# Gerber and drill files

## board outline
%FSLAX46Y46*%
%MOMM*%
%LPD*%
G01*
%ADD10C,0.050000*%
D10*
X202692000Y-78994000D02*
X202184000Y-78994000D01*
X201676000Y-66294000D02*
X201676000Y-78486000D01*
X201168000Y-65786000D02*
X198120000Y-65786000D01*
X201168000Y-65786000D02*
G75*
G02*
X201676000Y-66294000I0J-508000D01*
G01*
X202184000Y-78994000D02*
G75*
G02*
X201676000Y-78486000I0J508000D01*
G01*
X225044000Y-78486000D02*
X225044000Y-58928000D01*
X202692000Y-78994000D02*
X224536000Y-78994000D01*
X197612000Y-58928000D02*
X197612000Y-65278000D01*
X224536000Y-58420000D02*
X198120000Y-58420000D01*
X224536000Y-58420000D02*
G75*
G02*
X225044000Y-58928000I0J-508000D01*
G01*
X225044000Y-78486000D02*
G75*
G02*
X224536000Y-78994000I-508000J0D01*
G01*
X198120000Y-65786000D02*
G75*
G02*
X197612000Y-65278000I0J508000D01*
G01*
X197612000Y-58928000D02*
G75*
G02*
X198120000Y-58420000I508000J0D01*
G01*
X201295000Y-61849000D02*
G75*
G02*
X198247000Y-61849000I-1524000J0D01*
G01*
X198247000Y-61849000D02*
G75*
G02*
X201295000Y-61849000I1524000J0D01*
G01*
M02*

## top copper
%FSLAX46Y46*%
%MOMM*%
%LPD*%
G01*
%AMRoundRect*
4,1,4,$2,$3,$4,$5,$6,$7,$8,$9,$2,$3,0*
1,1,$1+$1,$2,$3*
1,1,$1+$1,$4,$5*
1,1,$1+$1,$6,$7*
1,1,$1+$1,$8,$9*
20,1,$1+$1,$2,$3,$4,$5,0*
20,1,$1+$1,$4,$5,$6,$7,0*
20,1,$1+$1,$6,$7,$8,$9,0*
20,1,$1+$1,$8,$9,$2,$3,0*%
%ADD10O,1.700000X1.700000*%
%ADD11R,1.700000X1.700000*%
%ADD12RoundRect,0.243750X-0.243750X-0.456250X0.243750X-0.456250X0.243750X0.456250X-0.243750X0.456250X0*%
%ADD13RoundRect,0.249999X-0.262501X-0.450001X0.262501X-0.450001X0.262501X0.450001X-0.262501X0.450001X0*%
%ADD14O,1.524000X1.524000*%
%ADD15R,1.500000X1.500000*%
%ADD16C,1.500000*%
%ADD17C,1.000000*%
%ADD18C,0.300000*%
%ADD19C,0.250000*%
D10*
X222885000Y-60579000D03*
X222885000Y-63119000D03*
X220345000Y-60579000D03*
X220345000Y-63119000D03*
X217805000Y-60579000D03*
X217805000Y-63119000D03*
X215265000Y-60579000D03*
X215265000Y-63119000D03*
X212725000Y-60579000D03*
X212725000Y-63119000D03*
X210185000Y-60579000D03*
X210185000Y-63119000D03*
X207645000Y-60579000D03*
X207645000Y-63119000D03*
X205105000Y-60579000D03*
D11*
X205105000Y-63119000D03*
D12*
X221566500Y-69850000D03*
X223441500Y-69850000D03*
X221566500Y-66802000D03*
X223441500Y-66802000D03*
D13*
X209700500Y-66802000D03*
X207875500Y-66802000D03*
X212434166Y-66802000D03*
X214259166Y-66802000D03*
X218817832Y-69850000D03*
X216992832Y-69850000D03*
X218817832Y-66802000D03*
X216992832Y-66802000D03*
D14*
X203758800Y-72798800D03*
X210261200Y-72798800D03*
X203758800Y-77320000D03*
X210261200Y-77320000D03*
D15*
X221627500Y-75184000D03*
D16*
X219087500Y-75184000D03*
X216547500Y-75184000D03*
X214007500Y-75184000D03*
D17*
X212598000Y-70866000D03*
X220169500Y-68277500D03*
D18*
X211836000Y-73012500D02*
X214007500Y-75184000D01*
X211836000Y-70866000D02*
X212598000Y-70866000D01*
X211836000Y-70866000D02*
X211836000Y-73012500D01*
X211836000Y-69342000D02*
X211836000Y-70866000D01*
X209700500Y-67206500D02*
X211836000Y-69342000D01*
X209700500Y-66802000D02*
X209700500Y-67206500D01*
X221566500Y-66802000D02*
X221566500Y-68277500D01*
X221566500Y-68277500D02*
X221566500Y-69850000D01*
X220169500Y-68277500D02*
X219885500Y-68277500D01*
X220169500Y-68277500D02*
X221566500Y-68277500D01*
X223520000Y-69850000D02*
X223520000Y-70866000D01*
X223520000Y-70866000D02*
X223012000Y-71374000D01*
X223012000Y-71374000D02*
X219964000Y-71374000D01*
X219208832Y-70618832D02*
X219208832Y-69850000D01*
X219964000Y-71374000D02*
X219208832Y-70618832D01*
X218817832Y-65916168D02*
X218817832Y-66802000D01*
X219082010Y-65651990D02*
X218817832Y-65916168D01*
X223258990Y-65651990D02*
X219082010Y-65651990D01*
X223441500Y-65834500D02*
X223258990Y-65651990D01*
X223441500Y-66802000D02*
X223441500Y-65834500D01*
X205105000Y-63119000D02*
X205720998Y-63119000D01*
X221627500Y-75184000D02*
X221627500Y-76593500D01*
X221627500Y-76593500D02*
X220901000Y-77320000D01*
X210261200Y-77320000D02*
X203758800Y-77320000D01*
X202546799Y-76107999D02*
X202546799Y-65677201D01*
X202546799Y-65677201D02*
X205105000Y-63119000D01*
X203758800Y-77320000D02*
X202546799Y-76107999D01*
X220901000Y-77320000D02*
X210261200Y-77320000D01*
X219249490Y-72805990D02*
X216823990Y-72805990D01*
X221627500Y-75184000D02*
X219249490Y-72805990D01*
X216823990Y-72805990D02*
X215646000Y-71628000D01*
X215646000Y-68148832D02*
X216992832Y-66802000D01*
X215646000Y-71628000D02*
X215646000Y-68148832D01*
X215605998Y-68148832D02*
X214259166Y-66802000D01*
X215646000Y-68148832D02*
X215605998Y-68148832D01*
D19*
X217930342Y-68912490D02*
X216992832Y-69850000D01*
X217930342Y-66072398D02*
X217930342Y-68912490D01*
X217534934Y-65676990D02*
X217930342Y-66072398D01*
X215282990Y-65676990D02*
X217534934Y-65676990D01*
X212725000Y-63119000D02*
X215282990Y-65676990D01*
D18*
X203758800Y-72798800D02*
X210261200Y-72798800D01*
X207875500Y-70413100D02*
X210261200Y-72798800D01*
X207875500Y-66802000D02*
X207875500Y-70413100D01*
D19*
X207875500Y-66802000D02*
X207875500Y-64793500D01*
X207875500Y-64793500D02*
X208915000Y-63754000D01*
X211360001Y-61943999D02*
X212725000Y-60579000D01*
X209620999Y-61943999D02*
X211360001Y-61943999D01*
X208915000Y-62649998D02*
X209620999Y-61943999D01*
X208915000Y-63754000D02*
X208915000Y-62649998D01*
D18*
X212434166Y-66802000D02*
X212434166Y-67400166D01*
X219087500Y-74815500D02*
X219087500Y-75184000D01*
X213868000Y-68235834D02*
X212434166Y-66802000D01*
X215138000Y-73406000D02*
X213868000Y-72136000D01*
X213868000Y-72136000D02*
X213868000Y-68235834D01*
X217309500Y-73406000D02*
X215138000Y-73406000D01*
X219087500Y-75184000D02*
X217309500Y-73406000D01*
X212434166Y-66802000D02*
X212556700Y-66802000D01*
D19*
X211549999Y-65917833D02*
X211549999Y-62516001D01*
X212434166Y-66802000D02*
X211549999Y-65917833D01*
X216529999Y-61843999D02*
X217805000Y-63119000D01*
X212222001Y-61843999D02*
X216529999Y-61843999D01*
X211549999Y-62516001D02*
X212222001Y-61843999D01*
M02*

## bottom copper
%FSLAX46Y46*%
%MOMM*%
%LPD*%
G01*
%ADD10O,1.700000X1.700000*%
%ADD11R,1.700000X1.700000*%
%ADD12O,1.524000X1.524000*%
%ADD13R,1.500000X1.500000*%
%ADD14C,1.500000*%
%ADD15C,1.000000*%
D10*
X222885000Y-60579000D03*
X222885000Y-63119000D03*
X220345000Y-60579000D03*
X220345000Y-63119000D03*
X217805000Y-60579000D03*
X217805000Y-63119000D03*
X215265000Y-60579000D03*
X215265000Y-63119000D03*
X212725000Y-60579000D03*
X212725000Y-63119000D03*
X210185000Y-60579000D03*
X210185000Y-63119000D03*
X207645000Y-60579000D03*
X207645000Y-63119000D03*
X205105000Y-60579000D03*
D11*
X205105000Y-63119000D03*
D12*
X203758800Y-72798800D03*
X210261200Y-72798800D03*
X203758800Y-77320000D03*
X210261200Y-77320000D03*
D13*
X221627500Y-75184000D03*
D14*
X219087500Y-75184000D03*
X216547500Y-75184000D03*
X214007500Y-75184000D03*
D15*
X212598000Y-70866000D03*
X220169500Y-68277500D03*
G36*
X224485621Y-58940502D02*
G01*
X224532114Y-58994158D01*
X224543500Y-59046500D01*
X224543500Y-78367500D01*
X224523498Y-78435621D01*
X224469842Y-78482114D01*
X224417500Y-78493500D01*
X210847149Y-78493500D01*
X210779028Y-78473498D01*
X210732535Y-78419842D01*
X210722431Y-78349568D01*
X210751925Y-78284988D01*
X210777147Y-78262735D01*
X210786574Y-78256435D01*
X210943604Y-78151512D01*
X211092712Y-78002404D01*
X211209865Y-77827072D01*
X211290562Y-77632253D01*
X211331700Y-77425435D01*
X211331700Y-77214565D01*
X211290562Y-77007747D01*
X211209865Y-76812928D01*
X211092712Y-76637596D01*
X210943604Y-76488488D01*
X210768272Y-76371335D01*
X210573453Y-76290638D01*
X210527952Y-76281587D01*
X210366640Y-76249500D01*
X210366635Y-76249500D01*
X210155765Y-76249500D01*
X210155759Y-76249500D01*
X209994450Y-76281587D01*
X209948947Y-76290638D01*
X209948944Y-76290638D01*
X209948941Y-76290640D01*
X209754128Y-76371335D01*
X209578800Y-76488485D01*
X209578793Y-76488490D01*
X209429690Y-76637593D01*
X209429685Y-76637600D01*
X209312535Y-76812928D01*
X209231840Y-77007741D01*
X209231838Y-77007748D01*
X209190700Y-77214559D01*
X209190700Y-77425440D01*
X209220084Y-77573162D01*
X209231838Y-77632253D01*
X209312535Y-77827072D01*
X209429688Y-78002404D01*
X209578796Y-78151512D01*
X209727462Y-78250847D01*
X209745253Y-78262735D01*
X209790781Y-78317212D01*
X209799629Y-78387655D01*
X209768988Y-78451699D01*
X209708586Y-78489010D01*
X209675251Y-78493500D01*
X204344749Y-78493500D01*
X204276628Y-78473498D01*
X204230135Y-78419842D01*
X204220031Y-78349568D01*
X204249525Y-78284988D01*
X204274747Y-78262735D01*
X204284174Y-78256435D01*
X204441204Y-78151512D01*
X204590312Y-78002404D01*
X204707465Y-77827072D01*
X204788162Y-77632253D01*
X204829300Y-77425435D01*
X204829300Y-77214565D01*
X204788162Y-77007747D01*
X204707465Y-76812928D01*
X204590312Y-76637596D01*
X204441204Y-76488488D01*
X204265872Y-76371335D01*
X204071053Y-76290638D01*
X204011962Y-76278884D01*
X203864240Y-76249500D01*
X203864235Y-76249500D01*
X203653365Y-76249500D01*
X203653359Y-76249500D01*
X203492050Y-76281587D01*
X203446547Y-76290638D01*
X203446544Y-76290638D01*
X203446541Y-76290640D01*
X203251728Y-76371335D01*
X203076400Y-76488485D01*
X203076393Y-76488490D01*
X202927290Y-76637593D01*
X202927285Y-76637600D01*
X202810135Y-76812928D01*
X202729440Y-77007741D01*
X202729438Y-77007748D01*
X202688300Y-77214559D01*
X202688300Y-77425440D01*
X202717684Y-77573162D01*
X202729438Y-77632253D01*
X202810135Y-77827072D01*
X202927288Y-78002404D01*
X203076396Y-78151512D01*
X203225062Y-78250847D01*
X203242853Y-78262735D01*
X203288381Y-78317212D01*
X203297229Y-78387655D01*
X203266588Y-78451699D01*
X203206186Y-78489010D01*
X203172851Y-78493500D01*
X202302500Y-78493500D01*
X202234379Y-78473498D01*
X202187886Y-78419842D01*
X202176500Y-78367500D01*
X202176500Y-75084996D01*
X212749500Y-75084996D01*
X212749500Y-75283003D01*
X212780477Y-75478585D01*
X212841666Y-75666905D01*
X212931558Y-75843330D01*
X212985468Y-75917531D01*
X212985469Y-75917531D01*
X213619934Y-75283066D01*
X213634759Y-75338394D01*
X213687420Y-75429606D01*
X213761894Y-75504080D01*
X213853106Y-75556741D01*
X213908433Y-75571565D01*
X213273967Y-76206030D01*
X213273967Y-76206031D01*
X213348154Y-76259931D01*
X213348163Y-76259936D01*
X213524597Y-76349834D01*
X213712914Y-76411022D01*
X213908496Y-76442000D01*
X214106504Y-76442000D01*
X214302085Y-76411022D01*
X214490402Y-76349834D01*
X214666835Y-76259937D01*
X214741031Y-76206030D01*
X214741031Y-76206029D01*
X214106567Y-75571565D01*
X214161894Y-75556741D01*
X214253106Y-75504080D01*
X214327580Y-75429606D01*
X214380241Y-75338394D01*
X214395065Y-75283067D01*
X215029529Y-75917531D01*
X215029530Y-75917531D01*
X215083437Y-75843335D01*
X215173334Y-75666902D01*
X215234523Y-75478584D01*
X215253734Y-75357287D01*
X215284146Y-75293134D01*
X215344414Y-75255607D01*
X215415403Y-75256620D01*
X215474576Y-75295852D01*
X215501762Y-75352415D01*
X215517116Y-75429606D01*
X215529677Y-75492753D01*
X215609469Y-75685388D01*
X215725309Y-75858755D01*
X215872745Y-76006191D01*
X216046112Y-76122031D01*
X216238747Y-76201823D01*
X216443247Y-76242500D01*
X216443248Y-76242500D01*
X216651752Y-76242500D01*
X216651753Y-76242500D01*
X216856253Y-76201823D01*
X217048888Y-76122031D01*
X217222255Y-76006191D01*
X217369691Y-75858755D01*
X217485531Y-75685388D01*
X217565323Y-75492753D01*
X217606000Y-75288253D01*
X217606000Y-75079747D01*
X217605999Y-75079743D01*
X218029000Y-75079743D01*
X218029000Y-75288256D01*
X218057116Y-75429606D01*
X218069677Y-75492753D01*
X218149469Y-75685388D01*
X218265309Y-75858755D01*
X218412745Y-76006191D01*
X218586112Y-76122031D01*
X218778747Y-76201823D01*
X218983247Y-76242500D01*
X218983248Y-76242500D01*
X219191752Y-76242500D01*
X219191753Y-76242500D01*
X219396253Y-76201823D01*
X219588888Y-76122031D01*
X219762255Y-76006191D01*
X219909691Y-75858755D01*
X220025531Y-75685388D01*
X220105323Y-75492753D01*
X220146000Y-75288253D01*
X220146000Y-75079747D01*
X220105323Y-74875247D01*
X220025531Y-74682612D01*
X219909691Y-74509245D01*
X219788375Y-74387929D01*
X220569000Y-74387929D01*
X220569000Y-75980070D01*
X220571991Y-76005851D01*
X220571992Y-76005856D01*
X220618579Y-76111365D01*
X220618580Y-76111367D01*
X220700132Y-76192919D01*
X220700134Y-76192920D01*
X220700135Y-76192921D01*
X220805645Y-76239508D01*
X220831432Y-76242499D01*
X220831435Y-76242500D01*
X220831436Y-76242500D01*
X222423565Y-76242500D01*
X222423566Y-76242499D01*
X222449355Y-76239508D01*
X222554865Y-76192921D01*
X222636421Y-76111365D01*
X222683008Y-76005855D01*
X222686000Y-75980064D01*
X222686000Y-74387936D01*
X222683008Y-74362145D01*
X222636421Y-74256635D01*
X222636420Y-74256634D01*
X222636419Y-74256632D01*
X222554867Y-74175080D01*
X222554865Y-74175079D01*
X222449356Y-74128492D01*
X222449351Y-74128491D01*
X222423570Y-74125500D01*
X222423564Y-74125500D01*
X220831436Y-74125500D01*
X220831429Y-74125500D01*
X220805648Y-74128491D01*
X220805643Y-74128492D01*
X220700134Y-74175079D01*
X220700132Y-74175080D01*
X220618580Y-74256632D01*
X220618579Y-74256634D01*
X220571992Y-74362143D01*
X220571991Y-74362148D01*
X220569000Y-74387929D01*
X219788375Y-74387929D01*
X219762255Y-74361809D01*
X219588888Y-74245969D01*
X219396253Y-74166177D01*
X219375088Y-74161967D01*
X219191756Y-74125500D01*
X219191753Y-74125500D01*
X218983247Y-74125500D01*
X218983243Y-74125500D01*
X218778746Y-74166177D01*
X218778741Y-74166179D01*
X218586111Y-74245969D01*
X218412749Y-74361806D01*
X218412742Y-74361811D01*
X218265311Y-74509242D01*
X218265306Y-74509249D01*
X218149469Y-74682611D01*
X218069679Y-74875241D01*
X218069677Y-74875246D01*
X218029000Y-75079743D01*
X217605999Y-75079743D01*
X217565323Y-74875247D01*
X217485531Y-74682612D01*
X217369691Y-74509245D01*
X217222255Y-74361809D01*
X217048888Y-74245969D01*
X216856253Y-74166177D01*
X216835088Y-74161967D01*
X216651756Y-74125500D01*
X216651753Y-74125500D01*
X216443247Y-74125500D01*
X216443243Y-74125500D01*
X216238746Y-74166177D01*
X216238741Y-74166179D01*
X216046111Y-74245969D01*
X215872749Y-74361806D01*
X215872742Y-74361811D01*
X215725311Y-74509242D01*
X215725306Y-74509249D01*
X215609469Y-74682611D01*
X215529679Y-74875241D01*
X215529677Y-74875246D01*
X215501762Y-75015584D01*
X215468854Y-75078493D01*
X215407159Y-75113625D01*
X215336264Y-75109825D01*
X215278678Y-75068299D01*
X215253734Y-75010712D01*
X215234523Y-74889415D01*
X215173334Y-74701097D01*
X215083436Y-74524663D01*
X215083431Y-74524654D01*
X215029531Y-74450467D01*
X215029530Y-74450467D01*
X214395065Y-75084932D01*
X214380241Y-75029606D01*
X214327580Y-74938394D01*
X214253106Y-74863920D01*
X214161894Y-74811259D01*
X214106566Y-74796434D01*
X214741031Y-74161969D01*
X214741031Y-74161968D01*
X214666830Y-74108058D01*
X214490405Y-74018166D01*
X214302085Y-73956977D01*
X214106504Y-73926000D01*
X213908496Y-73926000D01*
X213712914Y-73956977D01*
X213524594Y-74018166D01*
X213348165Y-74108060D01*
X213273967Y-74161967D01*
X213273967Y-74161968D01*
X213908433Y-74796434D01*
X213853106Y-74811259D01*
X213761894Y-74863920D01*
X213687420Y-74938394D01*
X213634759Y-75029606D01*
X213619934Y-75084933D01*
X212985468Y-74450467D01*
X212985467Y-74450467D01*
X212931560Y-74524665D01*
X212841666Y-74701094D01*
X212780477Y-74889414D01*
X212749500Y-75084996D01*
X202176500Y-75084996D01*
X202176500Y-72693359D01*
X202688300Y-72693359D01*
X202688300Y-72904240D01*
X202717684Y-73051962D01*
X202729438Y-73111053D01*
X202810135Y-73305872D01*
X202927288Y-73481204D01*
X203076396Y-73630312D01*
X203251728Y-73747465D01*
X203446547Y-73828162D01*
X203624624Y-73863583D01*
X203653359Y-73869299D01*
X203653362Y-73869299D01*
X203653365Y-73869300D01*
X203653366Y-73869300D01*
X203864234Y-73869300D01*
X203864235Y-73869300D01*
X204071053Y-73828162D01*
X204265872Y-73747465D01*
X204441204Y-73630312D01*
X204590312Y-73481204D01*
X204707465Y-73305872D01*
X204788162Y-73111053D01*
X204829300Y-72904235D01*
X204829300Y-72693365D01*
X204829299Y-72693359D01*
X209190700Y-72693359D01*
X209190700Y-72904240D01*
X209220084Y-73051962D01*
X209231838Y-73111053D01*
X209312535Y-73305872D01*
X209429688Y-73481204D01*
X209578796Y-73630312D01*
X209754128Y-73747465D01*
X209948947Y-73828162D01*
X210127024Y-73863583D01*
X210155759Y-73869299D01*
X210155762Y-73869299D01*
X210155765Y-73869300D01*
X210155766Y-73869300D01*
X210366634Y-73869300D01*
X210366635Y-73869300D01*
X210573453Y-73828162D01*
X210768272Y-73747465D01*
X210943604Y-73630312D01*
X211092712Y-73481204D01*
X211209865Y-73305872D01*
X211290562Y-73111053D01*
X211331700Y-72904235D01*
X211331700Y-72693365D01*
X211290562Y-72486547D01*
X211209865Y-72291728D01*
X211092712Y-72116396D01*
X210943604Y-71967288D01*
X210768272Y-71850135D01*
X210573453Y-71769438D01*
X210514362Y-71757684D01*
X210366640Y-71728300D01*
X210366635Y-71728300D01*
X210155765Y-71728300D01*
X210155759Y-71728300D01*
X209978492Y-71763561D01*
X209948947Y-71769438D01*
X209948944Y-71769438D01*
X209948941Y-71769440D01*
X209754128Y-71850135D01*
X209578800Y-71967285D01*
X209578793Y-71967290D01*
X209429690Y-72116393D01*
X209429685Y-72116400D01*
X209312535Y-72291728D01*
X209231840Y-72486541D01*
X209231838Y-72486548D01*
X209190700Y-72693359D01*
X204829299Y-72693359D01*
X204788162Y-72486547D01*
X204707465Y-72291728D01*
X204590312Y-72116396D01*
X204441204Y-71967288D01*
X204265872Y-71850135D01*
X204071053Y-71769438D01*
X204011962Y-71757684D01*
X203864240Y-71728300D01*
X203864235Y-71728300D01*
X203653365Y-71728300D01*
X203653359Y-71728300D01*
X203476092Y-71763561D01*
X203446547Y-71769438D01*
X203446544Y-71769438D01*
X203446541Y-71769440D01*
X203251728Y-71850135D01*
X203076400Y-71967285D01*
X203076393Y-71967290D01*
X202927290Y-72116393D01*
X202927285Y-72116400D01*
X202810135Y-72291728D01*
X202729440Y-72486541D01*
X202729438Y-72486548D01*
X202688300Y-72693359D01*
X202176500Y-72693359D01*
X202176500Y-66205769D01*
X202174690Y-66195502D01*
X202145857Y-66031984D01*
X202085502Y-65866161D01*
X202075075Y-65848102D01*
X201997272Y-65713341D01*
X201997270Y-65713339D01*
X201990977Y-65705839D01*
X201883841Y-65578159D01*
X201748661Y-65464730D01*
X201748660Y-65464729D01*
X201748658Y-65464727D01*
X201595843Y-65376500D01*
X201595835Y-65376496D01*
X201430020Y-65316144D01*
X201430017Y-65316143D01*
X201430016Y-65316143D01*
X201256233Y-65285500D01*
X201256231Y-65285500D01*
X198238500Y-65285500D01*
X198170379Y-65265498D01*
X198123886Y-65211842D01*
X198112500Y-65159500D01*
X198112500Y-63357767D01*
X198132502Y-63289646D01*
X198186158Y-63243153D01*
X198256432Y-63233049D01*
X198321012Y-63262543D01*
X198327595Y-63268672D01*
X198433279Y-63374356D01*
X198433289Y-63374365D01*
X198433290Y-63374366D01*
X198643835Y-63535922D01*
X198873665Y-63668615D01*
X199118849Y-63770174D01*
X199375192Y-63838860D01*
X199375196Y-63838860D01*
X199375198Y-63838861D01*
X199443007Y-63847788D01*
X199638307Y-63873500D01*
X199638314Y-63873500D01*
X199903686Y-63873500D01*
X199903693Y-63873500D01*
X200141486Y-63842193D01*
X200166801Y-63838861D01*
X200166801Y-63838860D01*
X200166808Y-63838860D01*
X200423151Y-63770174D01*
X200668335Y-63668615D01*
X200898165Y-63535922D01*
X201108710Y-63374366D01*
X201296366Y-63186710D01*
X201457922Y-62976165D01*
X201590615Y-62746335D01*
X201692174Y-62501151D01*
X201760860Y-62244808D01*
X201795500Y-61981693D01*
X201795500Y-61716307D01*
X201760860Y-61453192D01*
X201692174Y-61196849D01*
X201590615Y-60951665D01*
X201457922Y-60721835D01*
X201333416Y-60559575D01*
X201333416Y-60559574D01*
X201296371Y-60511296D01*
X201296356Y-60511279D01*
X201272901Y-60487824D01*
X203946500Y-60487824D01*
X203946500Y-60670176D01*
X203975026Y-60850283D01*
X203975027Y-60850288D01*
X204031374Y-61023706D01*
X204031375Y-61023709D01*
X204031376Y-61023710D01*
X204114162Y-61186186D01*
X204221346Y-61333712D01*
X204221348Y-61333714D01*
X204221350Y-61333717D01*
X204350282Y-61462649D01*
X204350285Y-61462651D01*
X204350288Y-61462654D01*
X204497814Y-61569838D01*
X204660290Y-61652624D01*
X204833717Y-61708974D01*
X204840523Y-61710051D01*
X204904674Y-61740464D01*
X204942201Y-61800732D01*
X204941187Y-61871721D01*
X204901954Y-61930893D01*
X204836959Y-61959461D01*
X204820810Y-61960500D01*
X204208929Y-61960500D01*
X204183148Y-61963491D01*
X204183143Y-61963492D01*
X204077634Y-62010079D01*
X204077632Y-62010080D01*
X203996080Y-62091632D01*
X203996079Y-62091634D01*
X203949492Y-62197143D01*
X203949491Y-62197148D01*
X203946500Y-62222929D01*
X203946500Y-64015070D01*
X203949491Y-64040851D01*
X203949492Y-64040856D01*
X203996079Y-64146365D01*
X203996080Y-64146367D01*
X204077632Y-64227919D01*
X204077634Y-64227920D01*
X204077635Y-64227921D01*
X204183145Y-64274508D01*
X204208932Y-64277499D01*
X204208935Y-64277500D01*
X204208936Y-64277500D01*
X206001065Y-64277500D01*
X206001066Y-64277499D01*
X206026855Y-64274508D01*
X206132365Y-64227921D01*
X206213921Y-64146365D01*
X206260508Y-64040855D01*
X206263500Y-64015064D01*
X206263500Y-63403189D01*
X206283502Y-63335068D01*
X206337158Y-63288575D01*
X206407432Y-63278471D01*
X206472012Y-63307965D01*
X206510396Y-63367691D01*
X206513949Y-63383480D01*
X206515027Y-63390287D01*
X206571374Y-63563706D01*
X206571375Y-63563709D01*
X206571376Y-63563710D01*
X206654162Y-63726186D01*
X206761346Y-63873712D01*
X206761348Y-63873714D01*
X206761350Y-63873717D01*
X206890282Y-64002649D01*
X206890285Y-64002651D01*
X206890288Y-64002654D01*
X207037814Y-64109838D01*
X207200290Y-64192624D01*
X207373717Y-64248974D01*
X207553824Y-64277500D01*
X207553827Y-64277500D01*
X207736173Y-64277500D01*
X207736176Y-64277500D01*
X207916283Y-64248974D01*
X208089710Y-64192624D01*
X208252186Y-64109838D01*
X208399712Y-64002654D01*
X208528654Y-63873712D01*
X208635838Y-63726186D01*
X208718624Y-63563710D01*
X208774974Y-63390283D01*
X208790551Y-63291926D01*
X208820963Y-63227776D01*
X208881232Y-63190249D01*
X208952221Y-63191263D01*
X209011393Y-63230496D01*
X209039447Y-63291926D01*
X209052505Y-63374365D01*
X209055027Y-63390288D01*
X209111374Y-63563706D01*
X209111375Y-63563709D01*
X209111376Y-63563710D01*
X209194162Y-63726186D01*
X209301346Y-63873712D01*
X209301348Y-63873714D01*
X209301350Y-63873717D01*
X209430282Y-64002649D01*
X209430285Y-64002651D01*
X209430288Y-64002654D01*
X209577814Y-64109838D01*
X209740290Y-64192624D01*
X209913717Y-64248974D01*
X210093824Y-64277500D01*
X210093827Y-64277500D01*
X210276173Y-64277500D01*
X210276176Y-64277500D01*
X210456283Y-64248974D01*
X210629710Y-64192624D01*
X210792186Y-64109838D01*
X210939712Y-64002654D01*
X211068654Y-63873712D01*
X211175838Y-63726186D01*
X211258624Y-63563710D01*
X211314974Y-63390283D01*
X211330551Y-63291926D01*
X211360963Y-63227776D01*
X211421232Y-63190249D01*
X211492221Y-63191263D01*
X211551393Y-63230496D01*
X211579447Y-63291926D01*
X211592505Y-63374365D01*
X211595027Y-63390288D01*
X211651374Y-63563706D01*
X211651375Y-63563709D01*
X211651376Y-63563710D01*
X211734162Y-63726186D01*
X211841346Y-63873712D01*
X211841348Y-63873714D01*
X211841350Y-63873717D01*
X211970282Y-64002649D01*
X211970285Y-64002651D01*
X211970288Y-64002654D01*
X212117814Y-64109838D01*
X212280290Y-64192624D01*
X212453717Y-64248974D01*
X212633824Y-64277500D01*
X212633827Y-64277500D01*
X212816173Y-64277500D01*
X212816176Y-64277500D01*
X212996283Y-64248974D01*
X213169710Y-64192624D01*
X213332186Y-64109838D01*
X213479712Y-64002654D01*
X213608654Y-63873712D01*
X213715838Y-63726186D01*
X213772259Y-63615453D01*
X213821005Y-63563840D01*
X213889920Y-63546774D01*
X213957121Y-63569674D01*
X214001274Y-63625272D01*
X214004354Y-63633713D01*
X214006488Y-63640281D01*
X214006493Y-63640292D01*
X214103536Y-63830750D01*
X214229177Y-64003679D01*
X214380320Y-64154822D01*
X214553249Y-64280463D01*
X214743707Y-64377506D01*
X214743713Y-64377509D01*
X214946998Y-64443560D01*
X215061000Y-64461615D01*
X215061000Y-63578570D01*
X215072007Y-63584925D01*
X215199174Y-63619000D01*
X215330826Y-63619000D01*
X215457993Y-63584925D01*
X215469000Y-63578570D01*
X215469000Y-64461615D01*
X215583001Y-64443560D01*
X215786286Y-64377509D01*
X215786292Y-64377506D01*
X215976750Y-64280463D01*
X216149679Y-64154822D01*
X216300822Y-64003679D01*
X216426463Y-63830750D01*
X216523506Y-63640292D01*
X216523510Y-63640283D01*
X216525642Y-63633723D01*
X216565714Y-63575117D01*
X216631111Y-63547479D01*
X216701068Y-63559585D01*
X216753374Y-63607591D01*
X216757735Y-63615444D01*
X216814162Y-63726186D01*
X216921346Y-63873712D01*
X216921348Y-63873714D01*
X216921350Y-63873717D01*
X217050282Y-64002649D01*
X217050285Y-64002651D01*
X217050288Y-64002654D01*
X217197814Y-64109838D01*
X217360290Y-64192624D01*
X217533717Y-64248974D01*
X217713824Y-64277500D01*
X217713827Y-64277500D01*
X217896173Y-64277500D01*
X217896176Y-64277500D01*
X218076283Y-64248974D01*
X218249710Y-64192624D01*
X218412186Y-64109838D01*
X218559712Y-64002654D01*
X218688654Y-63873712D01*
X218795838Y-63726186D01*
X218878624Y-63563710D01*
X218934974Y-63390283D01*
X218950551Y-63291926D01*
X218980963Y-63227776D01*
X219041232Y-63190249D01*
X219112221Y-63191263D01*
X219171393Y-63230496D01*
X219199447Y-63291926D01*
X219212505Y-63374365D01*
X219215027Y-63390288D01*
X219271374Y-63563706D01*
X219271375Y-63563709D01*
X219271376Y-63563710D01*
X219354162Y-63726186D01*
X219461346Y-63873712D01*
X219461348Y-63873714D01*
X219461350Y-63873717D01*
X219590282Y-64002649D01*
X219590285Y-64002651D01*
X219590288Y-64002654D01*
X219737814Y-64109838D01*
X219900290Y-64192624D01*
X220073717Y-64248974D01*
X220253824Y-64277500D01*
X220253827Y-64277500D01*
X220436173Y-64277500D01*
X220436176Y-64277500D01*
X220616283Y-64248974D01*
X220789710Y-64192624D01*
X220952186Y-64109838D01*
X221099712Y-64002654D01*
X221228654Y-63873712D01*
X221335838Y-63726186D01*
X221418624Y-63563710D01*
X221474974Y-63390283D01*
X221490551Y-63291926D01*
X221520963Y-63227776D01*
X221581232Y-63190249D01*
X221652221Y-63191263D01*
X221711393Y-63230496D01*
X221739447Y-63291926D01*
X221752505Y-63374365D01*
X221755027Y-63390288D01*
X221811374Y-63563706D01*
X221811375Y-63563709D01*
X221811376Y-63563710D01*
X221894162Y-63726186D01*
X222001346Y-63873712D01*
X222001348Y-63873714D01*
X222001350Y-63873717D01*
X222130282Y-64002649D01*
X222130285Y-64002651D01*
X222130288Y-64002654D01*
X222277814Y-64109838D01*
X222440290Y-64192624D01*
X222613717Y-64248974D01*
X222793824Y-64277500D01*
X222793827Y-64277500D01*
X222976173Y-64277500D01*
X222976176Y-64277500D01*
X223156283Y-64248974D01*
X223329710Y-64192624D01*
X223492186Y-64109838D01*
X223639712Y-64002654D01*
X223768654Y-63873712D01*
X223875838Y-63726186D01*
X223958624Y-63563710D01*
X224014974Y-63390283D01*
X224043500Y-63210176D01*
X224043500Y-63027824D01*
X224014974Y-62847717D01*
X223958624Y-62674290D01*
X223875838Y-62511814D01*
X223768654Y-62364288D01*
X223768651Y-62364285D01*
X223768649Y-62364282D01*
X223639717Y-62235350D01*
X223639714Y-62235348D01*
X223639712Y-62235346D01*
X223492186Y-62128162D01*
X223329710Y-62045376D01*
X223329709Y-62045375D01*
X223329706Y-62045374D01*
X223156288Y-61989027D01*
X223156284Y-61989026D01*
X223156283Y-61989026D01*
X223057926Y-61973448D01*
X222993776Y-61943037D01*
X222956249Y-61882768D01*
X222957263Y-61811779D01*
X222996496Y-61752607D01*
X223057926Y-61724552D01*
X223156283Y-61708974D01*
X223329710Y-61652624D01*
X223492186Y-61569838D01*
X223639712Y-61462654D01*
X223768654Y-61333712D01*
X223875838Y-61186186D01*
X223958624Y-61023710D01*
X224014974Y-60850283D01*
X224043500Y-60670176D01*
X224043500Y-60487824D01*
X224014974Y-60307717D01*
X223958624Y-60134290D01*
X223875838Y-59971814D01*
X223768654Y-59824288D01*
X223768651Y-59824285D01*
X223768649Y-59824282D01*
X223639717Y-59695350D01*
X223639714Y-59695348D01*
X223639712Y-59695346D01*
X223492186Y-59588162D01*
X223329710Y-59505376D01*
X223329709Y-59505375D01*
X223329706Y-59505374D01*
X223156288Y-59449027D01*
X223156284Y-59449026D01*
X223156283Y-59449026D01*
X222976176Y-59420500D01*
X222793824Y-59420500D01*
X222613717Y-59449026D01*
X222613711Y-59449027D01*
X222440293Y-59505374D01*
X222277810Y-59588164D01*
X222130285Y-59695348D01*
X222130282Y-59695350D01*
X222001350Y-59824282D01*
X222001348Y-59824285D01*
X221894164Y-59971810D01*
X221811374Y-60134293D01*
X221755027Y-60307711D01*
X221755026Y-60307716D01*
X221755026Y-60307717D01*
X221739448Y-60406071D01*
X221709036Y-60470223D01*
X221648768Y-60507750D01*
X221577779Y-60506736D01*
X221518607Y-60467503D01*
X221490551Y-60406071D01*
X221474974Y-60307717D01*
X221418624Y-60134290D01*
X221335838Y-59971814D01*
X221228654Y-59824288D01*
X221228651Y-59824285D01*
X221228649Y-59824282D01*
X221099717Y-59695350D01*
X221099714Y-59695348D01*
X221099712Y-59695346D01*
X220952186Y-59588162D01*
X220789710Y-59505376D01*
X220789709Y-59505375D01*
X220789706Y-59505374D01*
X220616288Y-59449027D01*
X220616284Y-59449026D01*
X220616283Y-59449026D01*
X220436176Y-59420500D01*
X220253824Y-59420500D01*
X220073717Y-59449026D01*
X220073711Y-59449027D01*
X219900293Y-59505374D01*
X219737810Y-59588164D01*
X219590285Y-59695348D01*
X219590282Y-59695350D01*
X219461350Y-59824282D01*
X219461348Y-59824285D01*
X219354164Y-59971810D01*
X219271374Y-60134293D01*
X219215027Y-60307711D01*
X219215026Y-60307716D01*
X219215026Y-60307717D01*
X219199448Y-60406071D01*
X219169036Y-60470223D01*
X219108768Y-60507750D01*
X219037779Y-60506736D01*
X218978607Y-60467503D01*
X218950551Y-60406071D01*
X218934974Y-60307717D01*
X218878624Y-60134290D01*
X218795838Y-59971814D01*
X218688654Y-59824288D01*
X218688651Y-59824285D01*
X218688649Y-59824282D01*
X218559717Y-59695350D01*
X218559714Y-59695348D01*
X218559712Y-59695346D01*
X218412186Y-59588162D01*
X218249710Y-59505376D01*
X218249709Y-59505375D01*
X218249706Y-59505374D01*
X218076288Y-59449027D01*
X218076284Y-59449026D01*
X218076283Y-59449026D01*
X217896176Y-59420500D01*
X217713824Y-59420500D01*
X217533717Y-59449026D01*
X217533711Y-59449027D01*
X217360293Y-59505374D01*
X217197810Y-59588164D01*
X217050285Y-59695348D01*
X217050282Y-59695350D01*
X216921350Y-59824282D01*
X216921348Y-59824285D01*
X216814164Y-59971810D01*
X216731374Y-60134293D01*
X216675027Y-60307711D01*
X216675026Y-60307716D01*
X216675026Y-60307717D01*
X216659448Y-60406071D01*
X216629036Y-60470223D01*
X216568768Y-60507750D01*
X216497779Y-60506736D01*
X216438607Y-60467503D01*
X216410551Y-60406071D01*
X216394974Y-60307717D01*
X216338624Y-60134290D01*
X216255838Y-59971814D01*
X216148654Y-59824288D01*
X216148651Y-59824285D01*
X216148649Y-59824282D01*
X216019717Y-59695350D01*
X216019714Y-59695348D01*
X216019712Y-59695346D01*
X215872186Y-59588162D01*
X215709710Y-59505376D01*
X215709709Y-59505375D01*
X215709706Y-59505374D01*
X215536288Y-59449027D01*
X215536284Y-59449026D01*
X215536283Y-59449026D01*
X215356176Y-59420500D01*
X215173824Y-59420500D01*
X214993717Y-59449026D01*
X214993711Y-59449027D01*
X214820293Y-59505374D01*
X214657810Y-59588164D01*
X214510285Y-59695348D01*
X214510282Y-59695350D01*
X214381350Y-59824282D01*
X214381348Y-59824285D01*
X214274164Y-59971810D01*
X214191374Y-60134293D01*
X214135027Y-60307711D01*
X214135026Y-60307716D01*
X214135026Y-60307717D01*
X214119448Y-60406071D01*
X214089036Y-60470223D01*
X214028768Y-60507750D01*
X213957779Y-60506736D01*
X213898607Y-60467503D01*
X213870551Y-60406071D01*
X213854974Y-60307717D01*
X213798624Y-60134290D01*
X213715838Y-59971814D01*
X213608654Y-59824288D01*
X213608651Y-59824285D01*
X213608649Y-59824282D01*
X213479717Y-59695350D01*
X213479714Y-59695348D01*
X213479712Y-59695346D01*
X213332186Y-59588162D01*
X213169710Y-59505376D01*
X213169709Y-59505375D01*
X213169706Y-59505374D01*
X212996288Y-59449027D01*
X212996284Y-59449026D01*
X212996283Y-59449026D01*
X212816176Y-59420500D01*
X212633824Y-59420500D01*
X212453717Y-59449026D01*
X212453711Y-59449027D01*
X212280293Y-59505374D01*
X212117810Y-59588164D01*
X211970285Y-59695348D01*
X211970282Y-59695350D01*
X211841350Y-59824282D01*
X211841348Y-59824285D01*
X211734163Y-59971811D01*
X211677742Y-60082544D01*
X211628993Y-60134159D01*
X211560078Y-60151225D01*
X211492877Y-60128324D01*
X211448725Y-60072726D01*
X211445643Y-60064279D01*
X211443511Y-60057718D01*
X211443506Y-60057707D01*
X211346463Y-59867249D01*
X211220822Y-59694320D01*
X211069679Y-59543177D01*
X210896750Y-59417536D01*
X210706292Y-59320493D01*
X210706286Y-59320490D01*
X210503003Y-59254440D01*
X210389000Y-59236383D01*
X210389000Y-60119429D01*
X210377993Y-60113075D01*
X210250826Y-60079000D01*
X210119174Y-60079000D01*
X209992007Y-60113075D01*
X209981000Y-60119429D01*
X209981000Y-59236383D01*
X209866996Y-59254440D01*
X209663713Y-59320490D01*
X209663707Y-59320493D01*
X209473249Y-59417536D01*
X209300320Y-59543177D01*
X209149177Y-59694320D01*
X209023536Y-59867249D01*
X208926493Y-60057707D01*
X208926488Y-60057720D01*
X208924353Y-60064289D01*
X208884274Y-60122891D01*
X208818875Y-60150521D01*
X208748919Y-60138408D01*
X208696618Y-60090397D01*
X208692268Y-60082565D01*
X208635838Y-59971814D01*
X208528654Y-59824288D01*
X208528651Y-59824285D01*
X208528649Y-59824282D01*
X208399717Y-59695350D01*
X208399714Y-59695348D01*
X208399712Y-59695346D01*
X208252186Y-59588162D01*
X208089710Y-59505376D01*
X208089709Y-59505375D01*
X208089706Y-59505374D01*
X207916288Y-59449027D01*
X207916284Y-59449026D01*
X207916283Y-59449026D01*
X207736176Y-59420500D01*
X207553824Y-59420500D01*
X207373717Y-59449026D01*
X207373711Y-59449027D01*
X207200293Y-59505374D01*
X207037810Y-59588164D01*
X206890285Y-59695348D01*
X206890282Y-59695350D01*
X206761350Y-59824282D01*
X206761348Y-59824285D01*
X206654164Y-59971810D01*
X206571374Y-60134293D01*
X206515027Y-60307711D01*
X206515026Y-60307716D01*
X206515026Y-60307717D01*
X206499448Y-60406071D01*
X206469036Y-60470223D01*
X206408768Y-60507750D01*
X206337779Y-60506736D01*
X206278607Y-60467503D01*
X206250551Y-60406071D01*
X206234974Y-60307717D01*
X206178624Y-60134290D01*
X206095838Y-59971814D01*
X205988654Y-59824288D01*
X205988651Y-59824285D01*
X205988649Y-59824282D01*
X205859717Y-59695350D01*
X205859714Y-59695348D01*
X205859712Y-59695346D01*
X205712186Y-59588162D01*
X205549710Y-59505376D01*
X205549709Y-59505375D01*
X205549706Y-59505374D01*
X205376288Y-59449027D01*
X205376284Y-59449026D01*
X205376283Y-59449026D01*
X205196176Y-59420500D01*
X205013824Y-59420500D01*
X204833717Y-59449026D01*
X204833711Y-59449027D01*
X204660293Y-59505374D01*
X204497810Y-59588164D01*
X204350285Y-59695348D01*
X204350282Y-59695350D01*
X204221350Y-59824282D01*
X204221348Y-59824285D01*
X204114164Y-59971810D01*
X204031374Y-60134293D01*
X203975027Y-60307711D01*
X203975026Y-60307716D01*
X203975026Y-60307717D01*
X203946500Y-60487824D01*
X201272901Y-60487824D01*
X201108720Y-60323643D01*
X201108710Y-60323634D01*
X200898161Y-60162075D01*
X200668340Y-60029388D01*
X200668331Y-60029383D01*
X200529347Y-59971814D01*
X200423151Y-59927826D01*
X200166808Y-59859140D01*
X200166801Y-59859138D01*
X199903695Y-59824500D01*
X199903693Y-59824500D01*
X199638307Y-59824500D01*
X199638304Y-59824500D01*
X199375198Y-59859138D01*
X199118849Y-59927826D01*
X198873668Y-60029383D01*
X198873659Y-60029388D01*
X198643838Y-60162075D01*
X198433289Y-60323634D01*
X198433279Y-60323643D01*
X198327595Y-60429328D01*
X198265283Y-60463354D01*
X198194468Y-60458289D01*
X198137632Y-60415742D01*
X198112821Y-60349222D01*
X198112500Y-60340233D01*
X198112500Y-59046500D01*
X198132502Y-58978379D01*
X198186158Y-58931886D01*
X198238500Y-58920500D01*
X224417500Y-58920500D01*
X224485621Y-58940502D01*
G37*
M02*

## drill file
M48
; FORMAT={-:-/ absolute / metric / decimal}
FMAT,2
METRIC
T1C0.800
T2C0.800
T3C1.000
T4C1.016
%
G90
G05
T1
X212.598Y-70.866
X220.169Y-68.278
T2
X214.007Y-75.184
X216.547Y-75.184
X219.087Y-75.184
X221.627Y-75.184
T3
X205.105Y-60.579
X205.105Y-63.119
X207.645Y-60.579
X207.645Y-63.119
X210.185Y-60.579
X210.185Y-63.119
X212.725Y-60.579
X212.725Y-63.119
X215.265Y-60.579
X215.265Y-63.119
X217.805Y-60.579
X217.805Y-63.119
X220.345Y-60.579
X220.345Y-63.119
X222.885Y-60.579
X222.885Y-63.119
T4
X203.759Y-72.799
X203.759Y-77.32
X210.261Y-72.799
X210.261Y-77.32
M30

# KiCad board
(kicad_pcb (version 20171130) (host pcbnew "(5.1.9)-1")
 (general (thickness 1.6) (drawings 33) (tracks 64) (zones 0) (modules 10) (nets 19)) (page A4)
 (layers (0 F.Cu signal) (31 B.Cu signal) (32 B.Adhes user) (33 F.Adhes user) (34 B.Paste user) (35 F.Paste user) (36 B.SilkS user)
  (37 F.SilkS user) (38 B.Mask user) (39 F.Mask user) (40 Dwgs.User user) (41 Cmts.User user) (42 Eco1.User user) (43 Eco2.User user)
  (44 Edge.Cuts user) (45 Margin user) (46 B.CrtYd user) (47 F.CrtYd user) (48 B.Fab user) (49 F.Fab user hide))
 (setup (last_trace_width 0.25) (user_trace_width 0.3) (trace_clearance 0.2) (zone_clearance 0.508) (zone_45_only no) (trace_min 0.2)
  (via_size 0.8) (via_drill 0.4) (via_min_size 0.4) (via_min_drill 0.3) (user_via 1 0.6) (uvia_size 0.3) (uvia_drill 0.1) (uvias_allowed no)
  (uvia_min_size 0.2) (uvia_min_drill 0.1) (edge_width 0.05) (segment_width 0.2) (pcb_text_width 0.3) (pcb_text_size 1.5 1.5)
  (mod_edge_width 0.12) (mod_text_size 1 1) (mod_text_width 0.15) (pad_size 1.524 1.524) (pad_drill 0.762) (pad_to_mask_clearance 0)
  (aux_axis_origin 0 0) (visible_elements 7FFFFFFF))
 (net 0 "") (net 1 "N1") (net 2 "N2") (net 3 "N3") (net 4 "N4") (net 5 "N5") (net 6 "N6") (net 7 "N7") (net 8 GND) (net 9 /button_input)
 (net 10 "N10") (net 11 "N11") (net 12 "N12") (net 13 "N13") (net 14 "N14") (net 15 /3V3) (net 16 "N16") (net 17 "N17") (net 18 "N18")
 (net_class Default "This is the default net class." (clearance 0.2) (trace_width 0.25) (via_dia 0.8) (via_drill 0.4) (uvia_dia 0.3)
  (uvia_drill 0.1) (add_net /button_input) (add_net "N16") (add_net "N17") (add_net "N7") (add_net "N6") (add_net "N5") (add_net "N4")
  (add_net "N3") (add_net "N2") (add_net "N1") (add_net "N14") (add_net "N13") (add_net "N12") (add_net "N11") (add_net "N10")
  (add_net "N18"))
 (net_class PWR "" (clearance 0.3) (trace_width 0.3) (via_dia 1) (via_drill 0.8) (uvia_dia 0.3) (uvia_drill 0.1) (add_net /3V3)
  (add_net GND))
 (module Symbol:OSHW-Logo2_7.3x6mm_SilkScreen (layer B.Cu) (at 207.01 73.66 180)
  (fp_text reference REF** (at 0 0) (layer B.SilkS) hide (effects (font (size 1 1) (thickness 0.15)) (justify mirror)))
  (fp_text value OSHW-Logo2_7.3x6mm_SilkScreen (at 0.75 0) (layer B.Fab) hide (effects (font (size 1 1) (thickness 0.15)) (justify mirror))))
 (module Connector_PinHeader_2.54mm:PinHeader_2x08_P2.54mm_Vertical (layer F.Cu) (at 205.105 63.119 90)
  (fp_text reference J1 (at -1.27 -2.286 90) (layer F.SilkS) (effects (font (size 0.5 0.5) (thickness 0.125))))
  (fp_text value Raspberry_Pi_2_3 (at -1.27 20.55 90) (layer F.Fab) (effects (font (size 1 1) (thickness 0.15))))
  (pad 16 thru_hole oval (at 2.54 17.78 90) (size 1.7 1.7) (drill 1) (layers *.Cu *.Mask) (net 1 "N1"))
  (pad 15 thru_hole oval (at 0 17.78 90) (size 1.7 1.7) (drill 1) (layers *.Cu *.Mask) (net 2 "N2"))
  (pad 14 thru_hole oval (at 2.54 15.24 90) (size 1.7 1.7) (drill 1) (layers *.Cu *.Mask) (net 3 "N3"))
  (pad 13 thru_hole oval (at 0 15.24 90) (size 1.7 1.7) (drill 1) (layers *.Cu *.Mask) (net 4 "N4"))
  (pad 12 thru_hole oval (at 2.54 12.7 90) (size 1.7 1.7) (drill 1) (layers *.Cu *.Mask) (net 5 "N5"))
  (pad 11 thru_hole oval (at 0 12.7 90) (size 1.7 1.7) (drill 1) (layers *.Cu *.Mask) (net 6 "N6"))
  (pad 10 thru_hole oval (at 2.54 10.16 90) (size 1.7 1.7) (drill 1) (layers *.Cu *.Mask) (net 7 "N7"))
  (pad 9 thru_hole oval (at 0 10.16 90) (size 1.7 1.7) (drill 1) (layers *.Cu *.Mask) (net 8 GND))
  (pad 8 thru_hole oval (at 2.54 7.62 90) (size 1.7 1.7) (drill 1) (layers *.Cu *.Mask) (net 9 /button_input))
  (pad 7 thru_hole oval (at 0 7.62 90) (size 1.7 1.7) (drill 1) (layers *.Cu *.Mask) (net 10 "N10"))
  (pad 6 thru_hole oval (at 2.54 5.08 90) (size 1.7 1.7) (drill 1) (layers *.Cu *.Mask) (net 8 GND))
  (pad 5 thru_hole oval (at 0 5.08 90) (size 1.7 1.7) (drill 1) (layers *.Cu *.Mask) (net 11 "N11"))
  (pad 4 thru_hole oval (at 2.54 2.54 90) (size 1.7 1.7) (drill 1) (layers *.Cu *.Mask) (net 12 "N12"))
  (pad 3 thru_hole oval (at 0 2.54 90) (size 1.7 1.7) (drill 1) (layers *.Cu *.Mask) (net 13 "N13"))
  (pad 2 thru_hole oval (at 2.54 0 90) (size 1.7 1.7) (drill 1) (layers *.Cu *.Mask) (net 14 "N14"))
  (pad 1 thru_hole rect (at 0 0 90) (size 1.7 1.7) (drill 1) (layers *.Cu *.Mask) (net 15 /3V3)))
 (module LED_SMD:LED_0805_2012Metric (layer F.Cu) (at 222.504 69.85)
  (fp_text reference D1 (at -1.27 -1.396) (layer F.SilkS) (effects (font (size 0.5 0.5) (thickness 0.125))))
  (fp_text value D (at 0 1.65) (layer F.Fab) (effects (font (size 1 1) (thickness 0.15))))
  (pad 1 smd roundrect (at -0.9375 0) (size 0.975 1.4) (layers F.Cu F.Paste F.Mask) (roundrect_rratio 0.25) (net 8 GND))
  (pad 2 smd roundrect (at 0.9375 0) (size 0.975 1.4) (layers F.Cu F.Paste F.Mask) (roundrect_rratio 0.25) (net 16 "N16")))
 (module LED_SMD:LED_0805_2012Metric (layer F.Cu) (at 222.504 66.802)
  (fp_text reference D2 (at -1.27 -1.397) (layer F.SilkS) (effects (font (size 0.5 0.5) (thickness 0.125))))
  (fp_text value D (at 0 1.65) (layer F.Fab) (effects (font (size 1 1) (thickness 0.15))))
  (pad 1 smd roundrect (at -0.9375 0) (size 0.975 1.4) (layers F.Cu F.Paste F.Mask) (roundrect_rratio 0.25) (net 8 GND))
  (pad 2 smd roundrect (at 0.9375 0) (size 0.975 1.4) (layers F.Cu F.Paste F.Mask) (roundrect_rratio 0.25) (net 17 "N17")))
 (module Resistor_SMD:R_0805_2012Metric (layer F.Cu) (at 208.788 66.802)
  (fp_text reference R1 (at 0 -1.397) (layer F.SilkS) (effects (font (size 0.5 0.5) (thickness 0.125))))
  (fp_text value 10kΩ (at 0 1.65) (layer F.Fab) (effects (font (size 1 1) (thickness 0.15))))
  (pad 2 smd roundrect (at 0.9125 0) (size 1.025 1.4) (layers F.Cu F.Paste F.Mask) (roundrect_rratio 0.2439014634146341) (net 8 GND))
  (pad 1 smd roundrect (at -0.9125 0) (size 1.025 1.4) (layers F.Cu F.Paste F.Mask) (roundrect_rratio 0.2439014634146341)
   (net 9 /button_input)))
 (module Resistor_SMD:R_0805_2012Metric (layer F.Cu) (at 213.346666 66.802)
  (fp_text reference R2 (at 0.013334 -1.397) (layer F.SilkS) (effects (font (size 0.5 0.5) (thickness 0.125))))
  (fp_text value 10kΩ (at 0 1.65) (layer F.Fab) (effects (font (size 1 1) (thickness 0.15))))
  (pad 1 smd roundrect (at -0.9125 0) (size 1.025 1.4) (layers F.Cu F.Paste F.Mask) (roundrect_rratio 0.2439014634146341) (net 6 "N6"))
  (pad 2 smd roundrect (at 0.9125 0) (size 1.025 1.4) (layers F.Cu F.Paste F.Mask) (roundrect_rratio 0.2439014634146341) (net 15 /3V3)))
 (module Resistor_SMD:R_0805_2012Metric (layer F.Cu) (at 217.905332 69.85)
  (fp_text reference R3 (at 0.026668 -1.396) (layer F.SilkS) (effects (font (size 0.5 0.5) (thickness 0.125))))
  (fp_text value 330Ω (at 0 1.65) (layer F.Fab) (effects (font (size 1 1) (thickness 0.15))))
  (pad 2 smd roundrect (at 0.9125 0) (size 1.025 1.4) (layers F.Cu F.Paste F.Mask) (roundrect_rratio 0.2439014634146341) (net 16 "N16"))
  (pad 1 smd roundrect (at -0.9125 0) (size 1.025 1.4) (layers F.Cu F.Paste F.Mask) (roundrect_rratio 0.2439014634146341) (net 10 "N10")))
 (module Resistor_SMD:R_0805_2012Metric (layer F.Cu) (at 217.905332 66.802)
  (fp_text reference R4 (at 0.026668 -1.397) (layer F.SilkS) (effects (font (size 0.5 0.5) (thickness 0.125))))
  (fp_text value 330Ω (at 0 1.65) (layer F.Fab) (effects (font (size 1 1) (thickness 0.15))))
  (pad 2 smd roundrect (at 0.9125 0) (size 1.025 1.4) (layers F.Cu F.Paste F.Mask) (roundrect_rratio 0.2439014634146341) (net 17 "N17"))
  (pad 1 smd roundrect (at -0.9125 0) (size 1.025 1.4) (layers F.Cu F.Paste F.Mask) (roundrect_rratio 0.2439014634146341) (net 15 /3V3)))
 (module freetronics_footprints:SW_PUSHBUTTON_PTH (layer F.Cu) (at 207.01 75.0594 180)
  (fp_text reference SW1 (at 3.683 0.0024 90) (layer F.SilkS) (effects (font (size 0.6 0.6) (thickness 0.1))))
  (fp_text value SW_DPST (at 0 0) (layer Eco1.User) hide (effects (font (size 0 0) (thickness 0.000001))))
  (pad 2 thru_hole oval (at 3.2512 2.2606 180) (size 1.524 1.524) (drill 1.016) (layers *.Cu *.Mask) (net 9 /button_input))
  (pad 2 thru_hole oval (at -3.2512 2.2606 180) (size 1.524 1.524) (drill 1.016) (layers *.Cu *.Mask) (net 9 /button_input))
  (pad 1 thru_hole oval (at 3.2512 -2.2606 180) (size 1.524 1.524) (drill 1.016) (layers *.Cu *.Mask) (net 15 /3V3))
  (pad 1 thru_hole oval (at -3.2512 -2.2606 180) (size 1.524 1.524) (drill 1.016) (layers *.Cu *.Mask) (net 15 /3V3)))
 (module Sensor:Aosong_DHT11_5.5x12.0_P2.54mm (layer F.Cu) (at 221.6275 75.184 270)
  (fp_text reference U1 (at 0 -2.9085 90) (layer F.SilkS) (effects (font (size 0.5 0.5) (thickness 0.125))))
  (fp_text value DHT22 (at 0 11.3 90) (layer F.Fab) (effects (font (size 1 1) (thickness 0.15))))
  (pad 1 thru_hole rect (at 0 0 270) (size 1.5 1.5) (drill 0.8) (layers *.Cu *.Mask) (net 15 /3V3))
  (pad 2 thru_hole circle (at 0 2.54 270) (size 1.5 1.5) (drill 0.8) (layers *.Cu *.Mask) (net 6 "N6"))
  (pad 3 thru_hole circle (at 0 5.08 270) (size 1.5 1.5) (drill 0.8) (layers *.Cu *.Mask) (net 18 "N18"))
  (pad 4 thru_hole circle (at 0 7.62 270) (size 1.5 1.5) (drill 0.8) (layers *.Cu *.Mask) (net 8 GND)))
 (gr_line (start 202.692 78.994) (end 202.184 78.994) (layer Edge.Cuts) (width 0.05))
 (gr_line (start 201.676 66.294) (end 201.676 78.486) (layer Edge.Cuts) (width 0.05))
 (gr_line (start 201.168 65.786) (end 198.12 65.786) (layer Edge.Cuts) (width 0.05))
 (gr_arc (start 201.168 66.294) (end 201.676 66.294) (angle -90) (layer Edge.Cuts) (width 0.05))
 (gr_arc (start 202.184 78.486) (end 201.676 78.486) (angle -90) (layer Edge.Cuts) (width 0.05))
 (gr_line (start 225.044 78.486) (end 225.044 58.928) (layer Edge.Cuts) (width 0.05))
 (gr_line (start 202.692 78.994) (end 224.536 78.994) (layer Edge.Cuts) (width 0.05))
 (gr_line (start 197.612 58.928) (end 197.612 65.278) (layer Edge.Cuts) (width 0.05))
 (gr_line (start 224.536 58.42) (end 198.12 58.42) (layer Edge.Cuts) (width 0.05))
 (gr_arc (start 224.536 58.928) (end 225.044 58.928) (angle -90) (layer Edge.Cuts) (width 0.05))
 (gr_arc (start 224.536 78.486) (end 224.536 78.994) (angle -90) (layer Edge.Cuts) (width 0.05))
 (gr_arc (start 198.12 65.278) (end 197.612 65.278) (angle -90) (layer Edge.Cuts) (width 0.05))
 (gr_arc (start 198.12 58.928) (end 198.12 58.42) (angle -90) (layer Edge.Cuts) (width 0.05))
 (gr_circle (center 199.771 61.849) (end 198.247 61.849) (layer Edge.Cuts) (width 0.05))
 (segment (start 211.836 73.0125) (end 214.0075 75.184) (width 0.3) (layer F.Cu) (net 8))
 (segment (start 211.836 70.866) (end 212.598 70.866) (width 0.3) (layer F.Cu) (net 8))
 (segment (start 211.836 70.866) (end 211.836 73.0125) (width 0.3) (layer F.Cu) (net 8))
 (via (at 212.598 70.866) (size 1) (drill 0.8) (layers F.Cu B.Cu) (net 8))
 (segment (start 211.836 69.342) (end 211.836 70.866) (width 0.3) (layer F.Cu) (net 8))
 (segment (start 209.7005 67.2065) (end 211.836 69.342) (width 0.3) (layer F.Cu) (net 8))
 (segment (start 209.7005 66.802) (end 209.7005 67.2065) (width 0.3) (layer F.Cu) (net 8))
 (segment (start 221.5665 66.802) (end 221.5665 68.2775) (width 0.3) (layer F.Cu) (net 8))
 (segment (start 221.5665 68.2775) (end 221.5665 69.85) (width 0.3) (layer F.Cu) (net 8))
 (segment (start 220.1695 68.2775) (end 219.8855 68.2775) (width 0.3) (layer F.Cu) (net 8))
 (via (at 220.1695 68.2775) (size 1) (drill 0.8) (layers F.Cu B.Cu) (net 8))
 (segment (start 220.1695 68.2775) (end 221.5665 68.2775) (width 0.3) (layer F.Cu) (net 8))
 (segment (start 223.52 69.85) (end 223.52 70.866) (width 0.3) (layer F.Cu) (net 16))
 (segment (start 223.52 70.866) (end 223.012 71.374) (width 0.3) (layer F.Cu) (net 16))
 (segment (start 223.012 71.374) (end 219.964 71.374) (width 0.3) (layer F.Cu) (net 16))
 (segment (start 219.208832 70.618832) (end 219.208832 69.85) (width 0.3) (layer F.Cu) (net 16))
 (segment (start 219.964 71.374) (end 219.208832 70.618832) (width 0.3) (layer F.Cu) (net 16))
 (segment (start 218.817832 65.916168) (end 218.817832 66.802) (width 0.3) (layer F.Cu) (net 17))
 (segment (start 219.08201 65.65199) (end 218.817832 65.916168) (width 0.3) (layer F.Cu) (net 17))
 (segment (start 223.25899 65.65199) (end 219.08201 65.65199) (width 0.3) (layer F.Cu) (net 17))
 (segment (start 223.4415 65.8345) (end 223.25899 65.65199) (width 0.3) (layer F.Cu) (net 17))
 (segment (start 223.4415 66.802) (end 223.4415 65.8345) (width 0.3) (layer F.Cu) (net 17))
 (segment (start 205.105 63.119) (end 205.720998 63.119) (width 0.3) (layer F.Cu) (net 15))
 (segment (start 221.6275 75.184) (end 221.6275 76.5935) (width 0.3) (layer F.Cu) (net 15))
 (segment (start 221.6275 76.5935) (end 220.901 77.32) (width 0.3) (layer F.Cu) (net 15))
 (segment (start 210.2612 77.32) (end 203.7588 77.32) (width 0.3) (layer F.Cu) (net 15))
 (segment (start 202.546799 76.107999) (end 202.546799 65.677201) (width 0.3) (layer F.Cu) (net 15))
 (segment (start 202.546799 65.677201) (end 205.105 63.119) (width 0.3) (layer F.Cu) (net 15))
 (segment (start 203.7588 77.32) (end 202.546799 76.107999) (width 0.3) (layer F.Cu) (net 15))
 (segment (start 220.901 77.32) (end 210.2612 77.32) (width 0.3) (layer F.Cu) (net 15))
 (segment (start 219.24949 72.80599) (end 216.82399 72.80599) (width 0.3) (layer F.Cu) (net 15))
 (segment (start 221.6275 75.184) (end 219.24949 72.80599) (width 0.3) (layer F.Cu) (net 15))
 (segment (start 216.82399 72.80599) (end 215.646 71.628) (width 0.3) (layer F.Cu) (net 15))
 (segment (start 215.646 68.148832) (end 216.992832 66.802) (width 0.3) (layer F.Cu) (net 15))
 (segment (start 215.646 71.628) (end 215.646 68.148832) (width 0.3) (layer F.Cu) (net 15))
 (segment (start 215.605998 68.148832) (end 214.259166 66.802) (width 0.3) (layer F.Cu) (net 15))
 (segment (start 215.646 68.148832) (end 215.605998 68.148832) (width 0.3) (layer F.Cu) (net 15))
 (segment (start 217.930342 68.91249) (end 216.992832 69.85) (width 0.25) (layer F.Cu) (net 10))
 (segment (start 217.930342 66.072398) (end 217.930342 68.91249) (width 0.25) (layer F.Cu) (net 10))
 (segment (start 217.534934 65.67699) (end 217.930342 66.072398) (width 0.25) (layer F.Cu) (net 10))
 (segment (start 215.28299 65.67699) (end 217.534934 65.67699) (width 0.25) (layer F.Cu) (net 10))
 (segment (start 212.725 63.119) (end 215.28299 65.67699) (width 0.25) (layer F.Cu) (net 10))
 (segment (start 203.7588 72.7988) (end 210.2612 72.7988) (width 0.3) (layer F.Cu) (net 9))
 (segment (start 207.8755 70.4131) (end 210.2612 72.7988) (width 0.3) (layer F.Cu) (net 9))
 (segment (start 207.8755 66.802) (end 207.8755 70.4131) (width 0.3) (layer F.Cu) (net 9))
 (segment (start 207.8755 66.802) (end 207.8755 64.7935) (width 0.25) (layer F.Cu) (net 9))
 (segment (start 207.8755 64.7935) (end 208.915 63.754) (width 0.25) (layer F.Cu) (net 9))
 (segment (start 211.360001 61.943999) (end 212.725 60.579) (width 0.25) (layer F.Cu) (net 9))
 (segment (start 209.620999 61.943999) (end 211.360001 61.943999) (width 0.25) (layer F.Cu) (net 9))
 (segment (start 208.915 62.649998) (end 209.620999 61.943999) (width 0.25) (layer F.Cu) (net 9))
 (segment (start 208.915 63.754) (end 208.915 62.649998) (width 0.25) (layer F.Cu) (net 9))
 (segment (start 212.434166 66.802) (end 212.434166 67.400166) (width 0.3) (layer F.Cu) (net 6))
 (segment (start 219.0875 74.8155) (end 219.0875 75.184) (width 0.3) (layer F.Cu) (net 6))
 (segment (start 213.868 68.235834) (end 212.434166 66.802) (width 0.3) (layer F.Cu) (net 6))
 (segment (start 215.138 73.406) (end 213.868 72.136) (width 0.3) (layer F.Cu) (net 6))
 (segment (start 213.868 72.136) (end 213.868 68.235834) (width 0.3) (layer F.Cu) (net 6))
 (segment (start 217.3095 73.406) (end 215.138 73.406) (width 0.3) (layer F.Cu) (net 6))
 (segment (start 219.0875 75.184) (end 217.3095 73.406) (width 0.3) (layer F.Cu) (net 6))
 (segment (start 212.434166 66.802) (end 212.5567 66.802) (width 0.3) (layer F.Cu) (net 6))
 (segment (start 211.549999 65.917833) (end 211.549999 62.516001) (width 0.25) (layer F.Cu) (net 6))
 (segment (start 212.434166 66.802) (end 211.549999 65.917833) (width 0.25) (layer F.Cu) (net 6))
 (segment (start 216.529999 61.843999) (end 217.805 63.119) (width 0.25) (layer F.Cu) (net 6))
 (segment (start 212.222001 61.843999) (end 216.529999 61.843999) (width 0.25) (layer F.Cu) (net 6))
 (segment (start 211.549999 62.516001) (end 212.222001 61.843999) (width 0.25) (layer F.Cu) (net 6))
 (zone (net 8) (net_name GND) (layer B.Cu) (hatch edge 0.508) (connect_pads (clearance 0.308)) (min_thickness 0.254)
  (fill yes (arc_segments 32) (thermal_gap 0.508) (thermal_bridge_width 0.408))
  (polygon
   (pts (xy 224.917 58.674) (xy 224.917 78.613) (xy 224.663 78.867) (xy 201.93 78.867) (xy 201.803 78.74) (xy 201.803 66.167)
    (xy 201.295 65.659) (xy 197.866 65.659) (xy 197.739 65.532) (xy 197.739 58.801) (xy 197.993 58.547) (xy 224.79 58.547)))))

